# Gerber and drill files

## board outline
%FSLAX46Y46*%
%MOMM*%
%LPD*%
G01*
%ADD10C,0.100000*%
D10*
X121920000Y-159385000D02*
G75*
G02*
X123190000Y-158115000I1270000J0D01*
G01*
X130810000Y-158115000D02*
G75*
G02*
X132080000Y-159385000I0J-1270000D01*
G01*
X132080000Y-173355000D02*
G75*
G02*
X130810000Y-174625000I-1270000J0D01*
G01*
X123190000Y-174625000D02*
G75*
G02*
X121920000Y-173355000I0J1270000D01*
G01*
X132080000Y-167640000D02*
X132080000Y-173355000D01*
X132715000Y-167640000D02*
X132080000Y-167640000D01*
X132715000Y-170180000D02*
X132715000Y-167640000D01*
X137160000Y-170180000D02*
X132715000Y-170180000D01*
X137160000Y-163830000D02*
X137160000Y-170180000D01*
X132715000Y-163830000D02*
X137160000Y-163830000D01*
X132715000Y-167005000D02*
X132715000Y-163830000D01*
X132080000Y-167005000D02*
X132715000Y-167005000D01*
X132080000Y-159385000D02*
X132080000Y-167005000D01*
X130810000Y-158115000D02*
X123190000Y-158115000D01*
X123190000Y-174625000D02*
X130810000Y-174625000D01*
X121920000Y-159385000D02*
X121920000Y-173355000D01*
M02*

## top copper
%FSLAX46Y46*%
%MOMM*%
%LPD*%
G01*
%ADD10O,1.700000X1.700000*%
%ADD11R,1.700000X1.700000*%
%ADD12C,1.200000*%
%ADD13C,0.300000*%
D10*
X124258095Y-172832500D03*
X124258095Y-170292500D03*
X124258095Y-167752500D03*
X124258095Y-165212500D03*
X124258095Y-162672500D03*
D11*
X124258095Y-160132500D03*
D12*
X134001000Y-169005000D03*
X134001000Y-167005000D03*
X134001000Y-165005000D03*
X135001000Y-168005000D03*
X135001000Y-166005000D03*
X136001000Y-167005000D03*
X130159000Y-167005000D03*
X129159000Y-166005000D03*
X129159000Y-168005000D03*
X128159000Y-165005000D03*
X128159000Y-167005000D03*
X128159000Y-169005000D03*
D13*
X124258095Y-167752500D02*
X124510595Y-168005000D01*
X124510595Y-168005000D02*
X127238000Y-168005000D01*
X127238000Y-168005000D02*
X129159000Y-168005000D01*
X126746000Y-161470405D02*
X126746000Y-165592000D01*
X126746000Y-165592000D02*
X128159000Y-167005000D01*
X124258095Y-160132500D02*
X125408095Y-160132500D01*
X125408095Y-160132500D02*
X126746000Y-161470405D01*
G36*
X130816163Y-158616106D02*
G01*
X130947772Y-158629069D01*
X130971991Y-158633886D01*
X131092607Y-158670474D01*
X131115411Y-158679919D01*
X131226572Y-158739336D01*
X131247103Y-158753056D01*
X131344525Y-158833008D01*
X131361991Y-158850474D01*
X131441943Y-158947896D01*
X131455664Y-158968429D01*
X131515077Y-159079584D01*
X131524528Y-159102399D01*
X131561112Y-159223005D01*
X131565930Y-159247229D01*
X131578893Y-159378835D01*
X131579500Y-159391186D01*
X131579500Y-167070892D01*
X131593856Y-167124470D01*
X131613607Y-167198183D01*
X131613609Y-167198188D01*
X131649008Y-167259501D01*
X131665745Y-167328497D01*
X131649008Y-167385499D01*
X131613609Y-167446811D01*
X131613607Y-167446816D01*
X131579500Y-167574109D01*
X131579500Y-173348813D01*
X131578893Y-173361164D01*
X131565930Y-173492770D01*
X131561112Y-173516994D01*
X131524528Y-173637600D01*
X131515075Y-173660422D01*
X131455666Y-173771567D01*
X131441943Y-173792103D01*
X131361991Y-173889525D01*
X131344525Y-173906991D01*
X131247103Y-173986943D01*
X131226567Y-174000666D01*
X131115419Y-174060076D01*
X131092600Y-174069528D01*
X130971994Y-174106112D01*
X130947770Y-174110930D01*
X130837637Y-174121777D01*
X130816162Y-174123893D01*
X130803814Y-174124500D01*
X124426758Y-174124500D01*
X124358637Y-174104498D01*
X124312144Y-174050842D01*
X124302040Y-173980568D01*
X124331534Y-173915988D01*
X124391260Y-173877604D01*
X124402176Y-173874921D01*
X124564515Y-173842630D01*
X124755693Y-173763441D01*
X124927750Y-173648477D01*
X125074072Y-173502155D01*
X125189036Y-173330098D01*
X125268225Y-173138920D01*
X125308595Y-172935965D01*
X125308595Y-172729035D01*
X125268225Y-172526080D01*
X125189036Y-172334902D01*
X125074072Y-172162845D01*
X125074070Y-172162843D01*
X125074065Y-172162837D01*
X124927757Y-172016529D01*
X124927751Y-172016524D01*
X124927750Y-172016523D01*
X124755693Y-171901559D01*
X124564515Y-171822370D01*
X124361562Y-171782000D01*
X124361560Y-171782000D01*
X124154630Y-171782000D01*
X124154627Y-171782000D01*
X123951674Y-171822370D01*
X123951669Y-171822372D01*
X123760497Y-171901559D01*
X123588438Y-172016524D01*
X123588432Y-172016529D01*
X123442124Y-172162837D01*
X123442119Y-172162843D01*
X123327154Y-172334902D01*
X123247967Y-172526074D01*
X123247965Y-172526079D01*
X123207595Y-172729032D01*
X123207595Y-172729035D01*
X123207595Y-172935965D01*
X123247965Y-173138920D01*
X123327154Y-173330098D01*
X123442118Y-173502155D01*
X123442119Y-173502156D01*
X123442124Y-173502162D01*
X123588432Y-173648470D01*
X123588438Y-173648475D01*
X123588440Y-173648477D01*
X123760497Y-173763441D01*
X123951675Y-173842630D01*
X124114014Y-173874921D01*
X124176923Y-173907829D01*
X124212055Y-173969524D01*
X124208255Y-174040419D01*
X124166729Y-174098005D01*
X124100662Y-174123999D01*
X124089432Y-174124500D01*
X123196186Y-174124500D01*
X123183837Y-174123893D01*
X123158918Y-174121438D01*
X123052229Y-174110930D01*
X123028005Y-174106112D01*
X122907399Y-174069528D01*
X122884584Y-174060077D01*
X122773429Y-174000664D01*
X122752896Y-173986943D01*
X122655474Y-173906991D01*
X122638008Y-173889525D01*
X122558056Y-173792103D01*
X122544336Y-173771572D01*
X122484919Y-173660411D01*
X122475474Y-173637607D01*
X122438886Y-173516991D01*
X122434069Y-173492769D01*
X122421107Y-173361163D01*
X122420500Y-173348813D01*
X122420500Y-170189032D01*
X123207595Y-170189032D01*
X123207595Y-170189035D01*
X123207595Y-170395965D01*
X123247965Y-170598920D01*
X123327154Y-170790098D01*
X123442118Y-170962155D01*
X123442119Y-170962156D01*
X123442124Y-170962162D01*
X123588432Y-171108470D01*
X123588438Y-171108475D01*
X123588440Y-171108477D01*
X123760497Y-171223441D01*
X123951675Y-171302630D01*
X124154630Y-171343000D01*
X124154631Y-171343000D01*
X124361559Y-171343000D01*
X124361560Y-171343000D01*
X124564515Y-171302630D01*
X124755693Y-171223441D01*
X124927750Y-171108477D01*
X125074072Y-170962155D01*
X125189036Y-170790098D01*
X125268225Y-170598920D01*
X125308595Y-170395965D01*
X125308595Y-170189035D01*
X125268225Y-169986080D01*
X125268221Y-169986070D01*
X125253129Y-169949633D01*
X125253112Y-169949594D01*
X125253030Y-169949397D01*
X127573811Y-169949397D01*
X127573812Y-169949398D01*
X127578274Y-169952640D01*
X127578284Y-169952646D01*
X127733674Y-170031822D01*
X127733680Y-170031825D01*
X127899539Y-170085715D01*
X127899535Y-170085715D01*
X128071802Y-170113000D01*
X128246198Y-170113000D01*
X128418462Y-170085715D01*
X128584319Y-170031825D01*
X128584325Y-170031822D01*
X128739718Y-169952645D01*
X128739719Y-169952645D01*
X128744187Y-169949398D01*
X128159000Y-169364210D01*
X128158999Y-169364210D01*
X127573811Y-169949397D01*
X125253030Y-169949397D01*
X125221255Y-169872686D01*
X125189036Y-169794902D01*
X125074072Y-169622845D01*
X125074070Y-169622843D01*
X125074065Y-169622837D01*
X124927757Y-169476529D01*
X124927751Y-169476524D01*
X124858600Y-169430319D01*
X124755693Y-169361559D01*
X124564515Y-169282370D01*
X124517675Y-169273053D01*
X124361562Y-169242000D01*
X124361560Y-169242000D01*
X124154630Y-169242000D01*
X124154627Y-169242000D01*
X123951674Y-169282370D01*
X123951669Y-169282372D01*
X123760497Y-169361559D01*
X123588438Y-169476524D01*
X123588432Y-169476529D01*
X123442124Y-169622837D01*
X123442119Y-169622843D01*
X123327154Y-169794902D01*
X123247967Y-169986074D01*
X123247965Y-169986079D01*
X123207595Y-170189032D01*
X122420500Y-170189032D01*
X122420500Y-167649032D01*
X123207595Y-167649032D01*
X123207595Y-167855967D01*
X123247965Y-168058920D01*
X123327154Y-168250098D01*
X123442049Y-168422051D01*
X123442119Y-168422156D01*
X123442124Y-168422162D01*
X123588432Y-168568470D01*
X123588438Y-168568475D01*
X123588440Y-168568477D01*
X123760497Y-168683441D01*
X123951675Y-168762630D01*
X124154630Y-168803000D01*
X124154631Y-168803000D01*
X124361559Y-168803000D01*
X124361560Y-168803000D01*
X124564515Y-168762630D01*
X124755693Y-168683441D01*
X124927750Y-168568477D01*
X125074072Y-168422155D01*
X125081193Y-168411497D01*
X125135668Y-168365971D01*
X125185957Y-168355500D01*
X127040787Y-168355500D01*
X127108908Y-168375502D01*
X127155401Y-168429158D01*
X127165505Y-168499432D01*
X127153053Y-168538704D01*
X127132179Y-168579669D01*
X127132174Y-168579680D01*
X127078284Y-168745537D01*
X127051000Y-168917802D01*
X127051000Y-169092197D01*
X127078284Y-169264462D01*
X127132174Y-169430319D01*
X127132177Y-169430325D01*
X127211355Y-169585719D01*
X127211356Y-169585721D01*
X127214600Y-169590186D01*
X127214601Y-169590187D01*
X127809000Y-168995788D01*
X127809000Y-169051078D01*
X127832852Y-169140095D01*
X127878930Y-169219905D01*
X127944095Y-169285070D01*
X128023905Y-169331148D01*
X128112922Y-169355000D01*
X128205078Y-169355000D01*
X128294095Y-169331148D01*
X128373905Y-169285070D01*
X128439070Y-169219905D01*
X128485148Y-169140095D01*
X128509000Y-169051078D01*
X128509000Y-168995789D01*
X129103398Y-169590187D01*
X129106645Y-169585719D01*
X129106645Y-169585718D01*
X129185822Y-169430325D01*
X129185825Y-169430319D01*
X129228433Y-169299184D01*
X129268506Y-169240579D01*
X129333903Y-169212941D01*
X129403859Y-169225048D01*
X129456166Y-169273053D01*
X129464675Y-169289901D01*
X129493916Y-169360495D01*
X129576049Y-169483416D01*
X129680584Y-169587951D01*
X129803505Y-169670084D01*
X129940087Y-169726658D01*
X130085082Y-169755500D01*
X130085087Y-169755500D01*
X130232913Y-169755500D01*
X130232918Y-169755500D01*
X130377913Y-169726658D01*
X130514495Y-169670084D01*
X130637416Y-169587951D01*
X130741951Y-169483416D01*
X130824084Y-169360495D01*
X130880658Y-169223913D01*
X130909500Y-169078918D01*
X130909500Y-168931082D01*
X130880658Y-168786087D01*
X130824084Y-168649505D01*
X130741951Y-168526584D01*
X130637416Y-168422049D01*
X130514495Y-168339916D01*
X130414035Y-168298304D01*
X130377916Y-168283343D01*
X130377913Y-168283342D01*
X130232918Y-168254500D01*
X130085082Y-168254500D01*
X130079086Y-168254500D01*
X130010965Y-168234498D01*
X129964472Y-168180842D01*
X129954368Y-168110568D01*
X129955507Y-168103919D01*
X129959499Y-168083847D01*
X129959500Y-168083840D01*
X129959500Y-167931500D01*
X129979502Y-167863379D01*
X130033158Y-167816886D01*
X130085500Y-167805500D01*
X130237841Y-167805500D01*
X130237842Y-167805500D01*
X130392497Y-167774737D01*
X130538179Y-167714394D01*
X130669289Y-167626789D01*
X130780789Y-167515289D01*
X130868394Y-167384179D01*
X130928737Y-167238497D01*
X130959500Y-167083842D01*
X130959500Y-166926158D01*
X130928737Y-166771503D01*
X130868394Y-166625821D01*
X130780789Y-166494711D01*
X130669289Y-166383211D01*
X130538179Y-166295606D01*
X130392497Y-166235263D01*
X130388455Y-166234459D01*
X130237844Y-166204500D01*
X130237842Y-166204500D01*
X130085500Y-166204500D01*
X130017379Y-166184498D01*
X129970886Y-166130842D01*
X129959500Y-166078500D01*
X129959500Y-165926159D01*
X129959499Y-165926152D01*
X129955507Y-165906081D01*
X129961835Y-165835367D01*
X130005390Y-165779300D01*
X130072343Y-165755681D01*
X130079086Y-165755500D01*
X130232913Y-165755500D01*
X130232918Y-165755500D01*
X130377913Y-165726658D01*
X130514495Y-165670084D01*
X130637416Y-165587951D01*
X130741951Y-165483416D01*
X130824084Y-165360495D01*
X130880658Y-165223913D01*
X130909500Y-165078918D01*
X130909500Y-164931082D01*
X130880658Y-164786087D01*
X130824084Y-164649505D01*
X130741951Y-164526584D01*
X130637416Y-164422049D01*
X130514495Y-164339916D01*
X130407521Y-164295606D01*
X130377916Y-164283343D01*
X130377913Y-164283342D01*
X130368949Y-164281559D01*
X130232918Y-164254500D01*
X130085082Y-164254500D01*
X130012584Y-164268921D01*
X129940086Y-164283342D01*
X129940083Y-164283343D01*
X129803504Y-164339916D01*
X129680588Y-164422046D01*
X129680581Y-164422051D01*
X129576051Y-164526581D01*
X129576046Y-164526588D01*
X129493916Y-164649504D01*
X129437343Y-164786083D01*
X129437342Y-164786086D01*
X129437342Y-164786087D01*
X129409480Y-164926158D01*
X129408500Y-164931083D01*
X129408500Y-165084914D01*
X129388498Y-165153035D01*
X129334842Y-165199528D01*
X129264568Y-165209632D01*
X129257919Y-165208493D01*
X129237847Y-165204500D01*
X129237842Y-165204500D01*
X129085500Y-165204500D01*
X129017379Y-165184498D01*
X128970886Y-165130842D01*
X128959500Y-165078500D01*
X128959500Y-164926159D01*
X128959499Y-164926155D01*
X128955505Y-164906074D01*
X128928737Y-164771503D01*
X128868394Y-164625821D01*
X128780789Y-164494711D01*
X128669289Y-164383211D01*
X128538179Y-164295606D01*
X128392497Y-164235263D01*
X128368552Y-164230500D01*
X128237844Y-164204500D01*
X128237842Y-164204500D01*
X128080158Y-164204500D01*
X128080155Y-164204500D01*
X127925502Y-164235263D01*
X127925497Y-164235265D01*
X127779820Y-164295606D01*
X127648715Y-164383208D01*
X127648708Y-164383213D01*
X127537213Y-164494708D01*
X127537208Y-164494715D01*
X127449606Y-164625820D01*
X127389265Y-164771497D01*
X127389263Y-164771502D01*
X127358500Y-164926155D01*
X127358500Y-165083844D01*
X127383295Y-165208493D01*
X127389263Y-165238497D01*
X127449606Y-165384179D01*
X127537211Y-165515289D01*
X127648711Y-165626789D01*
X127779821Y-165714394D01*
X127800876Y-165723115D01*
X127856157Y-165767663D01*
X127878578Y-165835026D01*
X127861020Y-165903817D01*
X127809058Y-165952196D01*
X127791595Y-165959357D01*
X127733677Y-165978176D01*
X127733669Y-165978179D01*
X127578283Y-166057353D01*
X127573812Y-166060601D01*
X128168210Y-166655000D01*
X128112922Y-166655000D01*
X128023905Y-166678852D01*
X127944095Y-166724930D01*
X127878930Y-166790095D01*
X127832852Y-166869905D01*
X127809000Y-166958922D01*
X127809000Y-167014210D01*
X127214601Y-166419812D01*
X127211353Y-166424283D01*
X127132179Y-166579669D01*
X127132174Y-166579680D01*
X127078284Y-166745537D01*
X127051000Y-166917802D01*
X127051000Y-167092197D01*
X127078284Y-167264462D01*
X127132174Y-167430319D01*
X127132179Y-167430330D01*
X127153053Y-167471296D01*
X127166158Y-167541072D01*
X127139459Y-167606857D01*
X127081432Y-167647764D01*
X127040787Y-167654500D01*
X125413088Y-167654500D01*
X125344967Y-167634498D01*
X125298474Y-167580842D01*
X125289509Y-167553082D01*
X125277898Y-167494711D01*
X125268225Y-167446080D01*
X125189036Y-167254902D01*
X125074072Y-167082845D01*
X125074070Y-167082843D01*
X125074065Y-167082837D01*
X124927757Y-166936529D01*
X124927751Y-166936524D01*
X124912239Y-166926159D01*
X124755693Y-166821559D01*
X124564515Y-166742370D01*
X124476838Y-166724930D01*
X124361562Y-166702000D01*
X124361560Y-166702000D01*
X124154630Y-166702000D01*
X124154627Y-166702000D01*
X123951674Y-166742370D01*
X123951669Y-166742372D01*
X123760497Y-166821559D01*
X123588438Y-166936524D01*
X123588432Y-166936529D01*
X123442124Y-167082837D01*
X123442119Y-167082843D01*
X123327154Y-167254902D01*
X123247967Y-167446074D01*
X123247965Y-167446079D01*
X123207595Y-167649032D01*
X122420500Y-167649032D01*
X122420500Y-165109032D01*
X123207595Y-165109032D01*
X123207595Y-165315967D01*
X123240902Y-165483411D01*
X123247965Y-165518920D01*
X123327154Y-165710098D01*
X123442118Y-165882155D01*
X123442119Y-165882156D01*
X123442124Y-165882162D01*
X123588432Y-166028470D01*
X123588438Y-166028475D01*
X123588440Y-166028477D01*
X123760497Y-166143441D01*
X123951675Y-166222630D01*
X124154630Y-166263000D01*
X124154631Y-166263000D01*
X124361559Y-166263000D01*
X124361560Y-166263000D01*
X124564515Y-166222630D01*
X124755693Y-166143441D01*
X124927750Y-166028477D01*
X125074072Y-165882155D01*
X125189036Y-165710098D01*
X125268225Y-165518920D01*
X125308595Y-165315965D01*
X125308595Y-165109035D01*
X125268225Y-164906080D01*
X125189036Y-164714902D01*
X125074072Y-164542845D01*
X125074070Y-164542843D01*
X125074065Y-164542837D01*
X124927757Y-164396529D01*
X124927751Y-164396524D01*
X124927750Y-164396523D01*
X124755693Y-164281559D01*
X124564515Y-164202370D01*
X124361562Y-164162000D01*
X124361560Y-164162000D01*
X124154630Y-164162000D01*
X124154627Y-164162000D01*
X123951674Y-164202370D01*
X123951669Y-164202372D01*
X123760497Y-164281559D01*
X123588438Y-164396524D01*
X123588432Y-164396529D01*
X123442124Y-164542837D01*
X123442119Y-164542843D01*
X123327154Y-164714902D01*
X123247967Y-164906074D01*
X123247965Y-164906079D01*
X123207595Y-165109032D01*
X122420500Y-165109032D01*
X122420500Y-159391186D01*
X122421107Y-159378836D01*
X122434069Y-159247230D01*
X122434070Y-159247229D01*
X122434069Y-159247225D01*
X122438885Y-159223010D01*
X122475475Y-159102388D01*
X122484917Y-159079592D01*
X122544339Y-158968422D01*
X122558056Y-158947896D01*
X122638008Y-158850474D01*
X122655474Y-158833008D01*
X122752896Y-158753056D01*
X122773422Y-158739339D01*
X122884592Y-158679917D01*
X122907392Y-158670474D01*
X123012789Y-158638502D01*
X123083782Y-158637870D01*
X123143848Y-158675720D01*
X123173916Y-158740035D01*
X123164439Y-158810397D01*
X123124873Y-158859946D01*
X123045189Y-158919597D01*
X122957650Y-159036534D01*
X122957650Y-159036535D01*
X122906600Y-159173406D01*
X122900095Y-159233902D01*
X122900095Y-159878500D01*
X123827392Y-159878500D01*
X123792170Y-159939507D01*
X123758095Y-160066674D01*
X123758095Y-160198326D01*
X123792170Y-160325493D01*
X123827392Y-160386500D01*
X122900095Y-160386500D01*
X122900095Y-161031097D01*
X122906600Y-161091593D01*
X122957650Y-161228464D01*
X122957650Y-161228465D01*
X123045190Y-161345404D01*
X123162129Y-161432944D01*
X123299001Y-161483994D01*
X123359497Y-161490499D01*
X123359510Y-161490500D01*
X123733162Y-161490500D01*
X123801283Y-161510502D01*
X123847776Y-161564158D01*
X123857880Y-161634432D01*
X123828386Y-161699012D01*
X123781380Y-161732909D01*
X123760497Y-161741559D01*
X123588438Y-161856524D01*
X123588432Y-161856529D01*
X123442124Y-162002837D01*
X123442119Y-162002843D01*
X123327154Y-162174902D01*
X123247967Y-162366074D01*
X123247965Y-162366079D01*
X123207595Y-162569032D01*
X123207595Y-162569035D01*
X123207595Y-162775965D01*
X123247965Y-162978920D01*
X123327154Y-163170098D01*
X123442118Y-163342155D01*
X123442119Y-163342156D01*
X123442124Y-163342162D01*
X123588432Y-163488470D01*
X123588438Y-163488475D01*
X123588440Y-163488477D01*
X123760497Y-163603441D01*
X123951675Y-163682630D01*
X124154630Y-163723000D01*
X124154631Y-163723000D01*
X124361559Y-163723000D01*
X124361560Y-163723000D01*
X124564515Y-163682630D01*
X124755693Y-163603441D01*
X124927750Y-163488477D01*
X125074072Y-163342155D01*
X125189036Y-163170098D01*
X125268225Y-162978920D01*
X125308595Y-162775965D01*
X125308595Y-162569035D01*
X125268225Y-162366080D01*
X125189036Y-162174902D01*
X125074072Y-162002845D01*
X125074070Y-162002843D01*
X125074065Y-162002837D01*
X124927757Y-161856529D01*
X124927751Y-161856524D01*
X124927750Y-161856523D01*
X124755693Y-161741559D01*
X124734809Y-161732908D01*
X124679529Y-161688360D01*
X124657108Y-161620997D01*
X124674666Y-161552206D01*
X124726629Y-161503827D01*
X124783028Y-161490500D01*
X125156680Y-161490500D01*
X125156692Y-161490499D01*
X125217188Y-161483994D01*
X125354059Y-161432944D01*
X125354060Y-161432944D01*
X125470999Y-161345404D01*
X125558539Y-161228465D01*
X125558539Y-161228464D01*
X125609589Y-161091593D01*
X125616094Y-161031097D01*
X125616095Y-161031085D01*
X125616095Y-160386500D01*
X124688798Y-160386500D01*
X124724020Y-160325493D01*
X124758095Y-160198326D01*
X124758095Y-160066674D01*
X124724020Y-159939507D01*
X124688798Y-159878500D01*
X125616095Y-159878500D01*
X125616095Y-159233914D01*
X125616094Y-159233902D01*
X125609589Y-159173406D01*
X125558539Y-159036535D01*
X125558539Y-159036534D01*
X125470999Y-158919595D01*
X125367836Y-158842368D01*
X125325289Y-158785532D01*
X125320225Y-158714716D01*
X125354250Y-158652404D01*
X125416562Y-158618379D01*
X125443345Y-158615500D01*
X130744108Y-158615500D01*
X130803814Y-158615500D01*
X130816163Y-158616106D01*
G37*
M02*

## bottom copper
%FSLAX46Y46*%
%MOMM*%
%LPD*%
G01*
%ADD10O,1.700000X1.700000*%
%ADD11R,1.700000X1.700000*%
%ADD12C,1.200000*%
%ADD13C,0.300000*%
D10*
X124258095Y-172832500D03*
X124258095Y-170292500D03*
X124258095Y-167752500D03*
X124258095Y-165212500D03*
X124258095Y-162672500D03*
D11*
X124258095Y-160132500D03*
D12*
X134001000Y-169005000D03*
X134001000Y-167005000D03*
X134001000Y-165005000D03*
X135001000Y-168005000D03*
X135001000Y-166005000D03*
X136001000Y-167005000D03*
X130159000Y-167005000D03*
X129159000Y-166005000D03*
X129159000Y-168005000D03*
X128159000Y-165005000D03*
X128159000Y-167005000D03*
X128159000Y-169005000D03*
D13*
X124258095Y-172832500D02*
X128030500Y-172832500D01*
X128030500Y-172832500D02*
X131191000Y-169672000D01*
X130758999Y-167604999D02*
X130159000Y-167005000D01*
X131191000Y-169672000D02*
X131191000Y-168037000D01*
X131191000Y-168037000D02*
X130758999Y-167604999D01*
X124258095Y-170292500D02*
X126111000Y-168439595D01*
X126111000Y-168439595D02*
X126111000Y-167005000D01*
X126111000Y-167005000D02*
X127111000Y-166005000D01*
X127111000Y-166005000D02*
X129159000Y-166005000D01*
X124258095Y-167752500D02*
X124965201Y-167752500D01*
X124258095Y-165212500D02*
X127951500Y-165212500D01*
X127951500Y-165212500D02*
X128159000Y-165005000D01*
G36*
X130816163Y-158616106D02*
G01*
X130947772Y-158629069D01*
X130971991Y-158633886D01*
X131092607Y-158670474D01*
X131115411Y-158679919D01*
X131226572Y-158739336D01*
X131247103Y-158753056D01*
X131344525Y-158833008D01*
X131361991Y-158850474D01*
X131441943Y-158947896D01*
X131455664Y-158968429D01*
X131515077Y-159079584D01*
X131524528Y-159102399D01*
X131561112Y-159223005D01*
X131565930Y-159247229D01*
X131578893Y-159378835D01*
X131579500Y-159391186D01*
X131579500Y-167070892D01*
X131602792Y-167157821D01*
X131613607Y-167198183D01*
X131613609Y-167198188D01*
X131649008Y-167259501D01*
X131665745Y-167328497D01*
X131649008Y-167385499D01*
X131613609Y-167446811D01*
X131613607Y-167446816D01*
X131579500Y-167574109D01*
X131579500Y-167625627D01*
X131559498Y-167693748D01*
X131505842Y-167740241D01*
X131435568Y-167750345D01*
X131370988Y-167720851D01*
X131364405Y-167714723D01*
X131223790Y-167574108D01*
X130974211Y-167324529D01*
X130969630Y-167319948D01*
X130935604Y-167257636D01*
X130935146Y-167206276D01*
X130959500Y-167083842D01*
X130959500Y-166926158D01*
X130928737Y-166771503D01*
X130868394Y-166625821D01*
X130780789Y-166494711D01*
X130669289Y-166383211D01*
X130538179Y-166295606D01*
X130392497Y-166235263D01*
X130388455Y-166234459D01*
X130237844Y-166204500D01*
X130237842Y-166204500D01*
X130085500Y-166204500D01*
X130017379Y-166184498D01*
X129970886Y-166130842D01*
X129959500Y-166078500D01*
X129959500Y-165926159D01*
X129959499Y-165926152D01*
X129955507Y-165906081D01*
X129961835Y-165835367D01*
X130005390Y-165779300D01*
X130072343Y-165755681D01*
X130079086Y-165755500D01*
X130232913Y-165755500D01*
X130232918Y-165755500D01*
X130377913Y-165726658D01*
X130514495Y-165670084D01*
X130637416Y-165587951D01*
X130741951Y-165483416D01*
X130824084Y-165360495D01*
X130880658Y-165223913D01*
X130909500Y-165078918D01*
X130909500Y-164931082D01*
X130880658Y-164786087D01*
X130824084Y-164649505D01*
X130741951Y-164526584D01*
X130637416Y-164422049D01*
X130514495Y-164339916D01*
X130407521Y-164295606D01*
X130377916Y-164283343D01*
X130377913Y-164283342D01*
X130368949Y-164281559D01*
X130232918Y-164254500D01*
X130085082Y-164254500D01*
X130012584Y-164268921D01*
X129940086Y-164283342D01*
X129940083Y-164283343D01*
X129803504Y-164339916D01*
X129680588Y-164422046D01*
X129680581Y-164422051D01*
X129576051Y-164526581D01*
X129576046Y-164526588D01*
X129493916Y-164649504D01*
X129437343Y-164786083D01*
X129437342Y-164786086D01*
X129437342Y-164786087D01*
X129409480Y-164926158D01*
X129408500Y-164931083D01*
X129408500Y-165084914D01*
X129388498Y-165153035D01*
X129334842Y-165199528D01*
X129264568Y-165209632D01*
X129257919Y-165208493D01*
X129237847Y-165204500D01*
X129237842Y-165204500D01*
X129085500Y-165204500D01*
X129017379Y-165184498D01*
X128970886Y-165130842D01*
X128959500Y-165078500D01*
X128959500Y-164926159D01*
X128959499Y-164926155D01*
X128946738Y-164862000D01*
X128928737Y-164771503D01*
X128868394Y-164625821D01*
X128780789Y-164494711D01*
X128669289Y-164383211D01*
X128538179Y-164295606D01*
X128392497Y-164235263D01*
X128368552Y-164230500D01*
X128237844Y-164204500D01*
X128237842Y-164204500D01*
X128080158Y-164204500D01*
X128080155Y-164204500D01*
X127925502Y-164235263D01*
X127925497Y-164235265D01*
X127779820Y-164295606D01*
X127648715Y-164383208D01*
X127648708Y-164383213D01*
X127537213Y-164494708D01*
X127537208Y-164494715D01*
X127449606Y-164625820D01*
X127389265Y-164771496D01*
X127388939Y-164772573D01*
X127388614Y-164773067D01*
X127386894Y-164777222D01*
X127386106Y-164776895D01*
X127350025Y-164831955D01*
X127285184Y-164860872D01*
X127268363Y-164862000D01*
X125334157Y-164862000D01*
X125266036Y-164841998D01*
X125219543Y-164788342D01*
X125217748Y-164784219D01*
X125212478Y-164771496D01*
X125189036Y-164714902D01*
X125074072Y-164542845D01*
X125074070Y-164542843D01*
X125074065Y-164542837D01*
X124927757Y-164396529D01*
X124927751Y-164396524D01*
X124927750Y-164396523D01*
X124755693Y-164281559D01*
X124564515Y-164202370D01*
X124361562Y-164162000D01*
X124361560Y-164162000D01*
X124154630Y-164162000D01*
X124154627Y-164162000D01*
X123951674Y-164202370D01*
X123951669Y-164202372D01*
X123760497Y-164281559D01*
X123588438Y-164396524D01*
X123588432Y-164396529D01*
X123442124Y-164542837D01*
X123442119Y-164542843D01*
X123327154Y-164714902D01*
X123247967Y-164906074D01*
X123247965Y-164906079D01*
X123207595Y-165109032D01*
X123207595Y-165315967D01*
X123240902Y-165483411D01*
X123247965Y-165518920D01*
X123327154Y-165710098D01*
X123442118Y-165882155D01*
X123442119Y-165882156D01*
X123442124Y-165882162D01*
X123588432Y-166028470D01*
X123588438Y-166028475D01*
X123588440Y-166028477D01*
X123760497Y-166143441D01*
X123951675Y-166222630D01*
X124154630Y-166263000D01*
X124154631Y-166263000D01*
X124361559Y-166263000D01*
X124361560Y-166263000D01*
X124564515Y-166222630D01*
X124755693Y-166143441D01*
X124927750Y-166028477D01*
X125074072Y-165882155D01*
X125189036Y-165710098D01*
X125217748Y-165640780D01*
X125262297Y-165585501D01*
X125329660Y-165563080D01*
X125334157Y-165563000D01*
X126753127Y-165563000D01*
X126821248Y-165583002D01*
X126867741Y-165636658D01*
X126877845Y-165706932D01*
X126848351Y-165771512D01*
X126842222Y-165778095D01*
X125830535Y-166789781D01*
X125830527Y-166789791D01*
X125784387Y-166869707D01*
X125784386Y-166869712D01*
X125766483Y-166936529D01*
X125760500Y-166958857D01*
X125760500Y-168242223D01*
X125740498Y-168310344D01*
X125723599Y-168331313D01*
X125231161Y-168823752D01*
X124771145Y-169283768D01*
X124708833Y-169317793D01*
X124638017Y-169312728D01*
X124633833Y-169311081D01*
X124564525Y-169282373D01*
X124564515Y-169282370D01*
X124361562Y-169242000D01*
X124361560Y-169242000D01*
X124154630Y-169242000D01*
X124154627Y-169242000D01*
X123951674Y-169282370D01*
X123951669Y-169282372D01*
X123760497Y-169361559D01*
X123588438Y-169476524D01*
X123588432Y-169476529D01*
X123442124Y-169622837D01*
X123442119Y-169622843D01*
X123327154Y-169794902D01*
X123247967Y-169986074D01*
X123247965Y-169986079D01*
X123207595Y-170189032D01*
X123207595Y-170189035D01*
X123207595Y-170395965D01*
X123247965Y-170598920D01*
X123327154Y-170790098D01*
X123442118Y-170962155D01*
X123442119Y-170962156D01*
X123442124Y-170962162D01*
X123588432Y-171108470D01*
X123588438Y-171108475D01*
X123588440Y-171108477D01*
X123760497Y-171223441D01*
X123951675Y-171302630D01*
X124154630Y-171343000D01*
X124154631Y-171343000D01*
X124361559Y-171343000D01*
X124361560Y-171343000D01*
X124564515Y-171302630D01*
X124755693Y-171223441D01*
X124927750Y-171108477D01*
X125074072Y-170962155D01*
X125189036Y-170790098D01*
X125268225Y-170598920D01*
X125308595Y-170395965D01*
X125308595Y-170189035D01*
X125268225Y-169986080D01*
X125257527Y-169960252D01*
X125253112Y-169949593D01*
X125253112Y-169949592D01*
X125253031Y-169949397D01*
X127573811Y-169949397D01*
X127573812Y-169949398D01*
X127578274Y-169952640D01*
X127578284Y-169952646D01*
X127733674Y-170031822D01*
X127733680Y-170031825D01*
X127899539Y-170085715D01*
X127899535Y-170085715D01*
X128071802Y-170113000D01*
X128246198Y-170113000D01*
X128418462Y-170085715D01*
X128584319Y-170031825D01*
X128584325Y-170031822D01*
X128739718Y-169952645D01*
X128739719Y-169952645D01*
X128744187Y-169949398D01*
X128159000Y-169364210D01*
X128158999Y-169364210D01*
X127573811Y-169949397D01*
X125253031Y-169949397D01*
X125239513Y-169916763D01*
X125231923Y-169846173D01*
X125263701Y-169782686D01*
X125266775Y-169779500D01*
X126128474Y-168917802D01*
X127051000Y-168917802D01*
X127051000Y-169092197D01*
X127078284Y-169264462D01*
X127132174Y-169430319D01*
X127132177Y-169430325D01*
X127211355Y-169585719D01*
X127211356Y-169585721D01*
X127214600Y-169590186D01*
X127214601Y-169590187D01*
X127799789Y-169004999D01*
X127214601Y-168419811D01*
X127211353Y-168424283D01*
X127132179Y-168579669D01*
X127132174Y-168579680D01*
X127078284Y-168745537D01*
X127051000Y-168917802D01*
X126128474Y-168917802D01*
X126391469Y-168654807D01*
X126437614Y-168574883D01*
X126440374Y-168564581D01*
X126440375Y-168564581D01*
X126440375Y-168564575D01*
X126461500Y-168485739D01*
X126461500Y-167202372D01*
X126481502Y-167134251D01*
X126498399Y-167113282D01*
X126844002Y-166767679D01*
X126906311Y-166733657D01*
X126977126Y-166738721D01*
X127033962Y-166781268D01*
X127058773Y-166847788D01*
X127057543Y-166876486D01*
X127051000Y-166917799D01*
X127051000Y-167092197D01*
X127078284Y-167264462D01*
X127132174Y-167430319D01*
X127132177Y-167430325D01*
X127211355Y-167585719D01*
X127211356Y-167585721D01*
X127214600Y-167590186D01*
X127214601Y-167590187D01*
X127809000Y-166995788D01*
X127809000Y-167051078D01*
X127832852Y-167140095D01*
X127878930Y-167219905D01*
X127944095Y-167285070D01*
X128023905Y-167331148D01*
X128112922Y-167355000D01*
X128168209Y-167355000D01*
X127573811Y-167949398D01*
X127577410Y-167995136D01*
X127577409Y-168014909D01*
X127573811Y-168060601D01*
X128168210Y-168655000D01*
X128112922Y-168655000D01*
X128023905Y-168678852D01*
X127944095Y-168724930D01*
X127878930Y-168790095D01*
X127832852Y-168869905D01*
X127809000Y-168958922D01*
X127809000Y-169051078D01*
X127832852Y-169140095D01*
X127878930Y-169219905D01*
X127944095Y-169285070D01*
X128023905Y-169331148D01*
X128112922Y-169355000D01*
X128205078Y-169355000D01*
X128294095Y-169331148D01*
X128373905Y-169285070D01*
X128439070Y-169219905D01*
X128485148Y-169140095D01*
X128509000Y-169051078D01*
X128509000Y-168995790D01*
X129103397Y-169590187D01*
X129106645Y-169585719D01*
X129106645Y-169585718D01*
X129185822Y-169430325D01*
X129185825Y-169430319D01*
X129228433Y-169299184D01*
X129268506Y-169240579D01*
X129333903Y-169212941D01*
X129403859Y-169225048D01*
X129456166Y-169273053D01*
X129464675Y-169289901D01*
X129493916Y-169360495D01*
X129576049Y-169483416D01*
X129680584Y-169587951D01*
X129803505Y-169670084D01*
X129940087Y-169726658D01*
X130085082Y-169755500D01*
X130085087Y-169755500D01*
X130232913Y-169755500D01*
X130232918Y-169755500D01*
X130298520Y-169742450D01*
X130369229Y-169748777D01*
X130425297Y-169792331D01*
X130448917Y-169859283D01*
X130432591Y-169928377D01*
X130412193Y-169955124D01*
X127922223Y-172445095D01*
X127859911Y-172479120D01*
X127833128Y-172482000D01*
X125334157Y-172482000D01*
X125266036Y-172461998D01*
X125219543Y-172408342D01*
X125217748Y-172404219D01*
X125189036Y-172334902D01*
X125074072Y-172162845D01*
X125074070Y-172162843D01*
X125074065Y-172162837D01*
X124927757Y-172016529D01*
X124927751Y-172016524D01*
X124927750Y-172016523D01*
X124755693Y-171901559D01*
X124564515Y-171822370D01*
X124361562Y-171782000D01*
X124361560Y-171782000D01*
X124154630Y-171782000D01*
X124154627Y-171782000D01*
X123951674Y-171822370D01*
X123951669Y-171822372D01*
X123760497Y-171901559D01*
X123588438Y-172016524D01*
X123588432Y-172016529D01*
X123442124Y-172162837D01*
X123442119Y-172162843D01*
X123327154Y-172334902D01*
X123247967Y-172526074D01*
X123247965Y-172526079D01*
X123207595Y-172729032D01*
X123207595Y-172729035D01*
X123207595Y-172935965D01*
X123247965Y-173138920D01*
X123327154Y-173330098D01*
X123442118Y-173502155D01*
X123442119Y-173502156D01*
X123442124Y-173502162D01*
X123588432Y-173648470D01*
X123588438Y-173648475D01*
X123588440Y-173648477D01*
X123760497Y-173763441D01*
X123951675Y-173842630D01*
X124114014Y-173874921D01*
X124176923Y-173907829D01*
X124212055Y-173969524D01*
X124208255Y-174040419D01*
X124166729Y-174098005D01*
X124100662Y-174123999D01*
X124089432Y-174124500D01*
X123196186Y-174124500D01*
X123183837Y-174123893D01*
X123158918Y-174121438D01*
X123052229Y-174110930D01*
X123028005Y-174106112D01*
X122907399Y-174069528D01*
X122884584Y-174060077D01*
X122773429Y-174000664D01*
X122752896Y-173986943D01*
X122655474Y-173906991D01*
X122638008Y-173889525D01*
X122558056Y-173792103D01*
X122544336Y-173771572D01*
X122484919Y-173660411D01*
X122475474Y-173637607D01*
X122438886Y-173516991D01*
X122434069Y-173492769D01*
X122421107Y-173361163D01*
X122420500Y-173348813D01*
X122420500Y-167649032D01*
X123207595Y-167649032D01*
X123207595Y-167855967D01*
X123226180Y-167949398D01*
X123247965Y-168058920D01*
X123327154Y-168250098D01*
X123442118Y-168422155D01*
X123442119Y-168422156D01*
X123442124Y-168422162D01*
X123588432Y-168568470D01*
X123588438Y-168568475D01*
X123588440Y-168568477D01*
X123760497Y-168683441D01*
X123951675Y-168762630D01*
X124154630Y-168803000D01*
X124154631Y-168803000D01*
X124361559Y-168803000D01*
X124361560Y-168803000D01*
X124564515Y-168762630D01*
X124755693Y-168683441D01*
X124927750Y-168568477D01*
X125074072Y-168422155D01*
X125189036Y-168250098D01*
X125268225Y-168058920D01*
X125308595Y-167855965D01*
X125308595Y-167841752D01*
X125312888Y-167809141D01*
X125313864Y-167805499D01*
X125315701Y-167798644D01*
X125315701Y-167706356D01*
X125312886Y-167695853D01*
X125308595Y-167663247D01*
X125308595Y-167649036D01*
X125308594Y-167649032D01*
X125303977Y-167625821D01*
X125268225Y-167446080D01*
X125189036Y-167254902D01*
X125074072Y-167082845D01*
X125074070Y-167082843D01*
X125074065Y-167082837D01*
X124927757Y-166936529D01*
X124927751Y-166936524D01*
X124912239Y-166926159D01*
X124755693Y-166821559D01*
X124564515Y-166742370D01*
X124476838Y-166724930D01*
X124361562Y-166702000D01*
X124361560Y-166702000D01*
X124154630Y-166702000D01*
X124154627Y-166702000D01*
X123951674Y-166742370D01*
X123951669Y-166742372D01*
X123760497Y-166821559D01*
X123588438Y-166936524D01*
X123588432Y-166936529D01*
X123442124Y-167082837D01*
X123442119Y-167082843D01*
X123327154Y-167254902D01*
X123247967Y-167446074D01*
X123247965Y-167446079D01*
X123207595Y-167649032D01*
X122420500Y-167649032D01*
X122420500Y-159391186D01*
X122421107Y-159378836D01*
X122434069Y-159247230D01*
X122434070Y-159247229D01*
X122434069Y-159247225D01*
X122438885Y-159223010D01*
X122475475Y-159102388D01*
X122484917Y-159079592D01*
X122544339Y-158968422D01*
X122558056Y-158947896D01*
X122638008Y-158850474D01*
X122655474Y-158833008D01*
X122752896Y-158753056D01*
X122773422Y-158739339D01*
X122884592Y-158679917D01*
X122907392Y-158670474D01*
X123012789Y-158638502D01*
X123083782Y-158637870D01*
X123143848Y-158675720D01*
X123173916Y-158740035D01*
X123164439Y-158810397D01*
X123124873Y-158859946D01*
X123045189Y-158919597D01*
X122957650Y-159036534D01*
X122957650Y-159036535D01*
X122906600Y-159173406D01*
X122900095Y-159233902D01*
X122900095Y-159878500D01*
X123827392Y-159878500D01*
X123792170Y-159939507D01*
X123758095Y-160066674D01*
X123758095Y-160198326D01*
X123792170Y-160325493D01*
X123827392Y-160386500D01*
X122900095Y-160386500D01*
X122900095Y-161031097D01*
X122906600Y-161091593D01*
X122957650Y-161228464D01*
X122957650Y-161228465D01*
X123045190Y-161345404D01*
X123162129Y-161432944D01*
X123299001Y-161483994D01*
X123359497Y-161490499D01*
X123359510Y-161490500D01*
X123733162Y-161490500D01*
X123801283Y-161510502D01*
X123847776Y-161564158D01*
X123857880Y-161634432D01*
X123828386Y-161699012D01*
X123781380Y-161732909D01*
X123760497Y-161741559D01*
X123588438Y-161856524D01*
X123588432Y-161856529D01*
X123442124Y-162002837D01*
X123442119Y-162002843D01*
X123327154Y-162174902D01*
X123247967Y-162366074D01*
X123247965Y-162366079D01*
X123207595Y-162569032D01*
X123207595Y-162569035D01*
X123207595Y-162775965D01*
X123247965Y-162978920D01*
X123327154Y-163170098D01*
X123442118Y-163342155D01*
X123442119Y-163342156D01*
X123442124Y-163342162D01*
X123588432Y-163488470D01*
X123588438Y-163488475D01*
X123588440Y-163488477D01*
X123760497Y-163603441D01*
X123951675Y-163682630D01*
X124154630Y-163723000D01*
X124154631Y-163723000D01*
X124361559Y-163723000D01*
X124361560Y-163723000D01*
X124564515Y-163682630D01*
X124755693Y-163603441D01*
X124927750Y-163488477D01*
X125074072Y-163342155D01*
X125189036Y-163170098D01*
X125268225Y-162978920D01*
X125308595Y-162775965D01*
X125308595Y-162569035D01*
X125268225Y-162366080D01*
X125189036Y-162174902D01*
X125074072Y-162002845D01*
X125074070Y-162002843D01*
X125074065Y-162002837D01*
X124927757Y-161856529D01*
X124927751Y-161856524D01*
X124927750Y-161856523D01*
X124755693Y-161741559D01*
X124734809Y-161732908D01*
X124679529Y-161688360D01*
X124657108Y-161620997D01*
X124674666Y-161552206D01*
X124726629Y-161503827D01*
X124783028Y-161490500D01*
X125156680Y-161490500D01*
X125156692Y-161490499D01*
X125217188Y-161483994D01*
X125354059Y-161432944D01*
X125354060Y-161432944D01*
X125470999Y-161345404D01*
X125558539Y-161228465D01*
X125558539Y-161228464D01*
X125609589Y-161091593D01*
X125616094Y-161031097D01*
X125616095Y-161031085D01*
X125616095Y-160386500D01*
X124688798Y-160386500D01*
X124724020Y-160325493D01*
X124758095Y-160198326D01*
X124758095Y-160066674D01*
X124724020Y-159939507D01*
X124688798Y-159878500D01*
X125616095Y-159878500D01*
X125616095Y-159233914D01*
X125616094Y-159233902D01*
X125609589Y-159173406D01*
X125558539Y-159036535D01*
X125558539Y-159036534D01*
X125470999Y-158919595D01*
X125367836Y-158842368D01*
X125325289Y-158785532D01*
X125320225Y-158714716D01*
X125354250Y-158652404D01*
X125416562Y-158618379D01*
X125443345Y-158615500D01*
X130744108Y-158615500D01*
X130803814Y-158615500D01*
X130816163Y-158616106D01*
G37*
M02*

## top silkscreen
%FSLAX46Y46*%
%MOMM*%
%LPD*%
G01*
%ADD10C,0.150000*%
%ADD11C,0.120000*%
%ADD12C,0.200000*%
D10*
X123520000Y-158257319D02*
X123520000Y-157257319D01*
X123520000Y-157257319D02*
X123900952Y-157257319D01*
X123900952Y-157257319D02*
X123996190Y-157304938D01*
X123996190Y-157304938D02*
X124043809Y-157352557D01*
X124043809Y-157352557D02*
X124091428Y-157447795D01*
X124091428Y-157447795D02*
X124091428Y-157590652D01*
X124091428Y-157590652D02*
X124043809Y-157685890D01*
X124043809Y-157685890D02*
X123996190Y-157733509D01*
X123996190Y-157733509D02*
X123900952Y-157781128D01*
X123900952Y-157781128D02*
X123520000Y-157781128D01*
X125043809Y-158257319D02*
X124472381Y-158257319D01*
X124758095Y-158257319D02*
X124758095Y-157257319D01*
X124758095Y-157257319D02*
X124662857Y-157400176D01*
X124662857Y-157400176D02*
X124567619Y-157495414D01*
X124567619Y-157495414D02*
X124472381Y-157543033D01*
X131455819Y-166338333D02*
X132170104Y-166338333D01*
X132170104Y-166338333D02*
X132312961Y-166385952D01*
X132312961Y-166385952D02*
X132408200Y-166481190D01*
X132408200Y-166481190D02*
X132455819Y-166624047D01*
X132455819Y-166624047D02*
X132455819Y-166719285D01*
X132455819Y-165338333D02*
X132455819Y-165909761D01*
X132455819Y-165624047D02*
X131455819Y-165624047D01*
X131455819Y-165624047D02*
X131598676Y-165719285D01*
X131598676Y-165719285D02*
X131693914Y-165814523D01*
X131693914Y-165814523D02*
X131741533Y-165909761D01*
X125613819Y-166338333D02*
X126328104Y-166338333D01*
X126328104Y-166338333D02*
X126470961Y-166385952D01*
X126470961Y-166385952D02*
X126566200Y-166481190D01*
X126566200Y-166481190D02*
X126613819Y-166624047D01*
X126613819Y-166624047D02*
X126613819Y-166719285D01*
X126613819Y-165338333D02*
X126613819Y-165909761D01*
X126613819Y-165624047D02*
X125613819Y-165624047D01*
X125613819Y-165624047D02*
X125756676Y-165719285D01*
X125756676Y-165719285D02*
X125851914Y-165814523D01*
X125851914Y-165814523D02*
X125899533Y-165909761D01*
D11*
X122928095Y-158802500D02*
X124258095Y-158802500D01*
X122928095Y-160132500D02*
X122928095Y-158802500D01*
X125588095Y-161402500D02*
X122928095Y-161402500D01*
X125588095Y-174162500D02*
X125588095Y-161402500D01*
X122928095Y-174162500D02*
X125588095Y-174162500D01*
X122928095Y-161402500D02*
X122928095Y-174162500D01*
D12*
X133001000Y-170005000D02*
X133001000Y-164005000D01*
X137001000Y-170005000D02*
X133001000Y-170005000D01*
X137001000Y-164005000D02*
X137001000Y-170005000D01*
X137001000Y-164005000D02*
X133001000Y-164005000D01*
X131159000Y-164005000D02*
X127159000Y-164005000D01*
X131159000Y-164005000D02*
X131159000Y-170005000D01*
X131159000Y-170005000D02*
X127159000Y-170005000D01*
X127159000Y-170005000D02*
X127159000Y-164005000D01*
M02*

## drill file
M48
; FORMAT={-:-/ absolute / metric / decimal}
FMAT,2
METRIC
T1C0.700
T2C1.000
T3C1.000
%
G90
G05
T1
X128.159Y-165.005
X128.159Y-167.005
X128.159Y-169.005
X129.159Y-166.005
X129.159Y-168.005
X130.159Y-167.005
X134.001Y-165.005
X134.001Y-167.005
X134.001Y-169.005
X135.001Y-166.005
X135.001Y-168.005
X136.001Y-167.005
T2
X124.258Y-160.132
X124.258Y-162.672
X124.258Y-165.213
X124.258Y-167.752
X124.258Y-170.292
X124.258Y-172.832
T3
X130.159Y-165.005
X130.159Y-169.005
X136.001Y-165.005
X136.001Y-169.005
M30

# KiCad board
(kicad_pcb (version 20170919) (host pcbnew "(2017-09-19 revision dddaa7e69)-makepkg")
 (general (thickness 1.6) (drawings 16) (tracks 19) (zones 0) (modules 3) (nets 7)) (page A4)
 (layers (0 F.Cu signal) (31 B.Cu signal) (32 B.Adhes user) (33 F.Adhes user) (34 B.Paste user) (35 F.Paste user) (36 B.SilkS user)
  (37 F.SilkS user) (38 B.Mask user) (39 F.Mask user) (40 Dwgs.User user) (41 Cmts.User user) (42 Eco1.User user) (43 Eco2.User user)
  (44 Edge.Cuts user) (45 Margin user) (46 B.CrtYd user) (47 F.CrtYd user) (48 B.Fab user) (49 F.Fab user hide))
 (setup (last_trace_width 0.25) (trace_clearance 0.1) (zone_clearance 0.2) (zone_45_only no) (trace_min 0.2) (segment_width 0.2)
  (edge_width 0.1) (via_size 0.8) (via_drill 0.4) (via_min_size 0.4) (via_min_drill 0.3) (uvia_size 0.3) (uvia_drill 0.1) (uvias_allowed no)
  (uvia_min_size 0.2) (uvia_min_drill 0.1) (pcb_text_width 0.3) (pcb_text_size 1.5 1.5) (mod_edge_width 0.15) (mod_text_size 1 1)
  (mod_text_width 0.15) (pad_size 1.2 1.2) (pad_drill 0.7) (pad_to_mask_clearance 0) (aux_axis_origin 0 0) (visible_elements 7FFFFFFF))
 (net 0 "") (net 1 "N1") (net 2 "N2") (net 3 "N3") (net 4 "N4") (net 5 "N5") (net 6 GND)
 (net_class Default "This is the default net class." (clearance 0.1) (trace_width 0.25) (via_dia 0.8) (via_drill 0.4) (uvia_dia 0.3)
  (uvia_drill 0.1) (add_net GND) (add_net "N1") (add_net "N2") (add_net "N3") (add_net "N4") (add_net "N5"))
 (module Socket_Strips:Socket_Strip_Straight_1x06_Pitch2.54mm (layer F.Cu) (at 124.258095 160.1325)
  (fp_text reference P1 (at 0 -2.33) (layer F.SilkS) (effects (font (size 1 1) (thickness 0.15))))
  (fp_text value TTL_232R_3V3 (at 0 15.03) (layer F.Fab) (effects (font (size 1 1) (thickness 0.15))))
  (fp_line (start -1.33 -1.33) (end 0 -1.33) (layer F.SilkS) (width 0.12))
  (fp_line (start -1.33 0) (end -1.33 -1.33) (layer F.SilkS) (width 0.12))
  (fp_line (start 1.33 1.27) (end -1.33 1.27) (layer F.SilkS) (width 0.12))
  (fp_line (start 1.33 14.03) (end 1.33 1.27) (layer F.SilkS) (width 0.12))
  (fp_line (start -1.33 14.03) (end 1.33 14.03) (layer F.SilkS) (width 0.12))
  (fp_line (start -1.33 1.27) (end -1.33 14.03) (layer F.SilkS) (width 0.12))
  (pad 6 thru_hole oval (at 0 12.7) (size 1.7 1.7) (drill 1) (layers *.Cu *.Mask) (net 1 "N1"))
  (pad 5 thru_hole oval (at 0 10.16) (size 1.7 1.7) (drill 1) (layers *.Cu *.Mask) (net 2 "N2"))
  (pad 4 thru_hole oval (at 0 7.62) (size 1.7 1.7) (drill 1) (layers *.Cu *.Mask) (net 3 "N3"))
  (pad 3 thru_hole oval (at 0 5.08) (size 1.7 1.7) (drill 1) (layers *.Cu *.Mask) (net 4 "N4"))
  (pad 2 thru_hole oval (at 0 2.54) (size 1.7 1.7) (drill 1) (layers *.Cu *.Mask) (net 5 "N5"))
  (pad 1 thru_hole rect (at 0 0) (size 1.7 1.7) (drill 1) (layers *.Cu *.Mask) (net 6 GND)))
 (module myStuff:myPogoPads (layer F.Cu) (at 135.001 167.005 270)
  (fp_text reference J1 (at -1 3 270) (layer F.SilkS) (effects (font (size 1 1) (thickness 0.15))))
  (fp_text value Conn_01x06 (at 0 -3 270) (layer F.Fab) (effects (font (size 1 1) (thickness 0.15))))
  (fp_line (start 3 2) (end -3 2) (layer F.SilkS) (width 0.2)) (fp_line (start 3 -2) (end 3 2) (layer F.SilkS) (width 0.2))
  (fp_line (start -3 -2) (end 3 -2) (layer F.SilkS) (width 0.2))
  (fp_line (start -3 -2) (end -3 2) (layer F.SilkS) (width 0.2))
  (pad "" np_thru_hole circle (at 2 -1 270) (size 1 1) (drill 1) (layers *.Cu *.Mask))
  (pad "" np_thru_hole circle (at -2 -1 270) (size 1 1) (drill 1) (layers *.Cu *.Mask))
  (pad 6 thru_hole circle (at 2 1 270) (size 1.2 1.2) (drill 0.7) (layers *.Cu *.Mask) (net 6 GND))
  (pad 5 thru_hole circle (at 0 1 270) (size 1.2 1.2) (drill 0.7) (layers *.Cu *.Mask) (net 6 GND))
  (pad 4 thru_hole circle (at -2 1 270) (size 1.2 1.2) (drill 0.7) (layers *.Cu *.Mask) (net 4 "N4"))
  (pad 3 thru_hole circle (at 1 0 270) (size 1.2 1.2) (drill 0.7) (layers *.Cu *.Mask) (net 3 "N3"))
  (pad 2 thru_hole circle (at -1 0 270) (size 1.2 1.2) (drill 0.7) (layers *.Cu *.Mask) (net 2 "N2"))
  (pad 1 thru_hole circle (at 0 -1 270) (size 1.2 1.2) (drill 0.7) (layers *.Cu *.Mask) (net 1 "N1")))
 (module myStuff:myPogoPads (layer F.Cu) (at 129.159 167.005 270)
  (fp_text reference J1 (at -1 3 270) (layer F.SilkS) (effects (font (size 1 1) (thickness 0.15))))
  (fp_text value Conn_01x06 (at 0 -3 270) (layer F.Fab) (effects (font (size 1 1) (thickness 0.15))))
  (fp_line (start -3 -2) (end -3 2) (layer F.SilkS) (width 0.2))
  (fp_line (start -3 -2) (end 3 -2) (layer F.SilkS) (width 0.2)) (fp_line (start 3 -2) (end 3 2) (layer F.SilkS) (width 0.2))
  (fp_line (start 3 2) (end -3 2) (layer F.SilkS) (width 0.2))
  (pad 1 thru_hole circle (at 0 -1 270) (size 1.2 1.2) (drill 0.7) (layers *.Cu *.Mask) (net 1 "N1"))
  (pad 2 thru_hole circle (at -1 0 270) (size 1.2 1.2) (drill 0.7) (layers *.Cu *.Mask) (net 2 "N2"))
  (pad 3 thru_hole circle (at 1 0 270) (size 1.2 1.2) (drill 0.7) (layers *.Cu *.Mask) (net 3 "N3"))
  (pad 4 thru_hole circle (at -2 1 270) (size 1.2 1.2) (drill 0.7) (layers *.Cu *.Mask) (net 4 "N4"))
  (pad 5 thru_hole circle (at 0 1 270) (size 1.2 1.2) (drill 0.7) (layers *.Cu *.Mask) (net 6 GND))
  (pad 6 thru_hole circle (at 2 1 270) (size 1.2 1.2) (drill 0.7) (layers *.Cu *.Mask) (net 6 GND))
  (pad "" np_thru_hole circle (at -2 -1 270) (size 1 1) (drill 1) (layers *.Cu *.Mask))
  (pad "" np_thru_hole circle (at 2 -1 270) (size 1 1) (drill 1) (layers *.Cu *.Mask)))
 (gr_arc (start 123.19 159.385) (end 123.19 158.115) (angle -90) (layer Edge.Cuts) (width 0.1))
 (gr_arc (start 130.81 159.385) (end 132.08 159.385) (angle -90) (layer Edge.Cuts) (width 0.1))
 (gr_arc (start 130.81 173.355) (end 130.81 174.625) (angle -90) (layer Edge.Cuts) (width 0.1))
 (gr_arc (start 123.19 173.355) (end 121.92 173.355) (angle -90) (layer Edge.Cuts) (width 0.1))
 (gr_line (start 132.08 167.64) (end 132.08 173.355) (layer Edge.Cuts) (width 0.1))
 (gr_line (start 132.715 167.64) (end 132.08 167.64) (layer Edge.Cuts) (width 0.1))
 (gr_line (start 132.715 170.18) (end 132.715 167.64) (layer Edge.Cuts) (width 0.1))
 (gr_line (start 137.16 170.18) (end 132.715 170.18) (layer Edge.Cuts) (width 0.1))
 (gr_line (start 137.16 163.83) (end 137.16 170.18) (layer Edge.Cuts) (width 0.1))
 (gr_line (start 132.715 163.83) (end 137.16 163.83) (layer Edge.Cuts) (width 0.1))
 (gr_line (start 132.715 167.005) (end 132.715 163.83) (layer Edge.Cuts) (width 0.1))
 (gr_line (start 132.08 167.005) (end 132.715 167.005) (layer Edge.Cuts) (width 0.1))
 (gr_line (start 132.08 159.385) (end 132.08 167.005) (layer Edge.Cuts) (width 0.1))
 (gr_line (start 130.81 158.115) (end 123.19 158.115) (layer Edge.Cuts) (width 0.1))
 (gr_line (start 123.19 174.625) (end 130.81 174.625) (layer Edge.Cuts) (width 0.1))
 (gr_line (start 121.92 159.385) (end 121.92 173.355) (layer Edge.Cuts) (width 0.1))
 (segment (start 124.258095 172.8325) (end 128.0305 172.8325) (width 0.3) (layer B.Cu) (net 1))
 (segment (start 128.0305 172.8325) (end 131.191 169.672) (width 0.3) (layer B.Cu) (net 1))
 (segment (start 130.758999 167.604999) (end 130.159 167.005) (width 0.3) (layer B.Cu) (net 1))
 (segment (start 131.191 169.672) (end 131.191 168.037) (width 0.3) (layer B.Cu) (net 1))
 (segment (start 131.191 168.037) (end 130.758999 167.604999) (width 0.3) (layer B.Cu) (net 1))
 (segment (start 124.258095 170.2925) (end 126.111 168.439595) (width 0.3) (layer B.Cu) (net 2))
 (segment (start 126.111 168.439595) (end 126.111 167.005) (width 0.3) (layer B.Cu) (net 2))
 (segment (start 126.111 167.005) (end 127.111 166.005) (width 0.3) (layer B.Cu) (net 2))
 (segment (start 127.111 166.005) (end 129.159 166.005) (width 0.3) (layer B.Cu) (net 2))
 (segment (start 124.258095 167.7525) (end 124.510595 168.005) (width 0.3) (layer F.Cu) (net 3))
 (segment (start 124.510595 168.005) (end 127.238 168.005) (width 0.3) (layer F.Cu) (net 3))
 (segment (start 127.238 168.005) (end 129.159 168.005) (width 0.3) (layer F.Cu) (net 3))
 (segment (start 124.258095 167.7525) (end 124.965201 167.7525) (width 0.3) (layer B.Cu) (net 3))
 (segment (start 124.258095 165.2125) (end 127.9515 165.2125) (width 0.3) (layer B.Cu) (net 4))
 (segment (start 127.9515 165.2125) (end 128.159 165.005) (width 0.3) (layer B.Cu) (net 4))
 (segment (start 126.746 161.470405) (end 126.746 165.592) (width 0.3) (layer F.Cu) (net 6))
 (segment (start 126.746 165.592) (end 128.159 167.005) (width 0.3) (layer F.Cu) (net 6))
 (segment (start 124.258095 160.1325) (end 125.408095 160.1325) (width 0.3) (layer F.Cu) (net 6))
 (segment (start 125.408095 160.1325) (end 126.746 161.470405) (width 0.3) (layer F.Cu) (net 6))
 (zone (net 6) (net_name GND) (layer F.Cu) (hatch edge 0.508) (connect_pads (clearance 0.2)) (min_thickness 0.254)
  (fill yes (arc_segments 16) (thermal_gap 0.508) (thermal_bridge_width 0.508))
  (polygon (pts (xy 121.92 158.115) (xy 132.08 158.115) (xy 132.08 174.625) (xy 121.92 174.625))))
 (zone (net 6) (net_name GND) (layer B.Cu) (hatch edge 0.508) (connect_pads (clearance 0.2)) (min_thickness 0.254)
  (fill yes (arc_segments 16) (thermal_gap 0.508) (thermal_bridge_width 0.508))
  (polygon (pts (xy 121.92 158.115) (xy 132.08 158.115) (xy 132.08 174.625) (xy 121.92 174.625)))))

